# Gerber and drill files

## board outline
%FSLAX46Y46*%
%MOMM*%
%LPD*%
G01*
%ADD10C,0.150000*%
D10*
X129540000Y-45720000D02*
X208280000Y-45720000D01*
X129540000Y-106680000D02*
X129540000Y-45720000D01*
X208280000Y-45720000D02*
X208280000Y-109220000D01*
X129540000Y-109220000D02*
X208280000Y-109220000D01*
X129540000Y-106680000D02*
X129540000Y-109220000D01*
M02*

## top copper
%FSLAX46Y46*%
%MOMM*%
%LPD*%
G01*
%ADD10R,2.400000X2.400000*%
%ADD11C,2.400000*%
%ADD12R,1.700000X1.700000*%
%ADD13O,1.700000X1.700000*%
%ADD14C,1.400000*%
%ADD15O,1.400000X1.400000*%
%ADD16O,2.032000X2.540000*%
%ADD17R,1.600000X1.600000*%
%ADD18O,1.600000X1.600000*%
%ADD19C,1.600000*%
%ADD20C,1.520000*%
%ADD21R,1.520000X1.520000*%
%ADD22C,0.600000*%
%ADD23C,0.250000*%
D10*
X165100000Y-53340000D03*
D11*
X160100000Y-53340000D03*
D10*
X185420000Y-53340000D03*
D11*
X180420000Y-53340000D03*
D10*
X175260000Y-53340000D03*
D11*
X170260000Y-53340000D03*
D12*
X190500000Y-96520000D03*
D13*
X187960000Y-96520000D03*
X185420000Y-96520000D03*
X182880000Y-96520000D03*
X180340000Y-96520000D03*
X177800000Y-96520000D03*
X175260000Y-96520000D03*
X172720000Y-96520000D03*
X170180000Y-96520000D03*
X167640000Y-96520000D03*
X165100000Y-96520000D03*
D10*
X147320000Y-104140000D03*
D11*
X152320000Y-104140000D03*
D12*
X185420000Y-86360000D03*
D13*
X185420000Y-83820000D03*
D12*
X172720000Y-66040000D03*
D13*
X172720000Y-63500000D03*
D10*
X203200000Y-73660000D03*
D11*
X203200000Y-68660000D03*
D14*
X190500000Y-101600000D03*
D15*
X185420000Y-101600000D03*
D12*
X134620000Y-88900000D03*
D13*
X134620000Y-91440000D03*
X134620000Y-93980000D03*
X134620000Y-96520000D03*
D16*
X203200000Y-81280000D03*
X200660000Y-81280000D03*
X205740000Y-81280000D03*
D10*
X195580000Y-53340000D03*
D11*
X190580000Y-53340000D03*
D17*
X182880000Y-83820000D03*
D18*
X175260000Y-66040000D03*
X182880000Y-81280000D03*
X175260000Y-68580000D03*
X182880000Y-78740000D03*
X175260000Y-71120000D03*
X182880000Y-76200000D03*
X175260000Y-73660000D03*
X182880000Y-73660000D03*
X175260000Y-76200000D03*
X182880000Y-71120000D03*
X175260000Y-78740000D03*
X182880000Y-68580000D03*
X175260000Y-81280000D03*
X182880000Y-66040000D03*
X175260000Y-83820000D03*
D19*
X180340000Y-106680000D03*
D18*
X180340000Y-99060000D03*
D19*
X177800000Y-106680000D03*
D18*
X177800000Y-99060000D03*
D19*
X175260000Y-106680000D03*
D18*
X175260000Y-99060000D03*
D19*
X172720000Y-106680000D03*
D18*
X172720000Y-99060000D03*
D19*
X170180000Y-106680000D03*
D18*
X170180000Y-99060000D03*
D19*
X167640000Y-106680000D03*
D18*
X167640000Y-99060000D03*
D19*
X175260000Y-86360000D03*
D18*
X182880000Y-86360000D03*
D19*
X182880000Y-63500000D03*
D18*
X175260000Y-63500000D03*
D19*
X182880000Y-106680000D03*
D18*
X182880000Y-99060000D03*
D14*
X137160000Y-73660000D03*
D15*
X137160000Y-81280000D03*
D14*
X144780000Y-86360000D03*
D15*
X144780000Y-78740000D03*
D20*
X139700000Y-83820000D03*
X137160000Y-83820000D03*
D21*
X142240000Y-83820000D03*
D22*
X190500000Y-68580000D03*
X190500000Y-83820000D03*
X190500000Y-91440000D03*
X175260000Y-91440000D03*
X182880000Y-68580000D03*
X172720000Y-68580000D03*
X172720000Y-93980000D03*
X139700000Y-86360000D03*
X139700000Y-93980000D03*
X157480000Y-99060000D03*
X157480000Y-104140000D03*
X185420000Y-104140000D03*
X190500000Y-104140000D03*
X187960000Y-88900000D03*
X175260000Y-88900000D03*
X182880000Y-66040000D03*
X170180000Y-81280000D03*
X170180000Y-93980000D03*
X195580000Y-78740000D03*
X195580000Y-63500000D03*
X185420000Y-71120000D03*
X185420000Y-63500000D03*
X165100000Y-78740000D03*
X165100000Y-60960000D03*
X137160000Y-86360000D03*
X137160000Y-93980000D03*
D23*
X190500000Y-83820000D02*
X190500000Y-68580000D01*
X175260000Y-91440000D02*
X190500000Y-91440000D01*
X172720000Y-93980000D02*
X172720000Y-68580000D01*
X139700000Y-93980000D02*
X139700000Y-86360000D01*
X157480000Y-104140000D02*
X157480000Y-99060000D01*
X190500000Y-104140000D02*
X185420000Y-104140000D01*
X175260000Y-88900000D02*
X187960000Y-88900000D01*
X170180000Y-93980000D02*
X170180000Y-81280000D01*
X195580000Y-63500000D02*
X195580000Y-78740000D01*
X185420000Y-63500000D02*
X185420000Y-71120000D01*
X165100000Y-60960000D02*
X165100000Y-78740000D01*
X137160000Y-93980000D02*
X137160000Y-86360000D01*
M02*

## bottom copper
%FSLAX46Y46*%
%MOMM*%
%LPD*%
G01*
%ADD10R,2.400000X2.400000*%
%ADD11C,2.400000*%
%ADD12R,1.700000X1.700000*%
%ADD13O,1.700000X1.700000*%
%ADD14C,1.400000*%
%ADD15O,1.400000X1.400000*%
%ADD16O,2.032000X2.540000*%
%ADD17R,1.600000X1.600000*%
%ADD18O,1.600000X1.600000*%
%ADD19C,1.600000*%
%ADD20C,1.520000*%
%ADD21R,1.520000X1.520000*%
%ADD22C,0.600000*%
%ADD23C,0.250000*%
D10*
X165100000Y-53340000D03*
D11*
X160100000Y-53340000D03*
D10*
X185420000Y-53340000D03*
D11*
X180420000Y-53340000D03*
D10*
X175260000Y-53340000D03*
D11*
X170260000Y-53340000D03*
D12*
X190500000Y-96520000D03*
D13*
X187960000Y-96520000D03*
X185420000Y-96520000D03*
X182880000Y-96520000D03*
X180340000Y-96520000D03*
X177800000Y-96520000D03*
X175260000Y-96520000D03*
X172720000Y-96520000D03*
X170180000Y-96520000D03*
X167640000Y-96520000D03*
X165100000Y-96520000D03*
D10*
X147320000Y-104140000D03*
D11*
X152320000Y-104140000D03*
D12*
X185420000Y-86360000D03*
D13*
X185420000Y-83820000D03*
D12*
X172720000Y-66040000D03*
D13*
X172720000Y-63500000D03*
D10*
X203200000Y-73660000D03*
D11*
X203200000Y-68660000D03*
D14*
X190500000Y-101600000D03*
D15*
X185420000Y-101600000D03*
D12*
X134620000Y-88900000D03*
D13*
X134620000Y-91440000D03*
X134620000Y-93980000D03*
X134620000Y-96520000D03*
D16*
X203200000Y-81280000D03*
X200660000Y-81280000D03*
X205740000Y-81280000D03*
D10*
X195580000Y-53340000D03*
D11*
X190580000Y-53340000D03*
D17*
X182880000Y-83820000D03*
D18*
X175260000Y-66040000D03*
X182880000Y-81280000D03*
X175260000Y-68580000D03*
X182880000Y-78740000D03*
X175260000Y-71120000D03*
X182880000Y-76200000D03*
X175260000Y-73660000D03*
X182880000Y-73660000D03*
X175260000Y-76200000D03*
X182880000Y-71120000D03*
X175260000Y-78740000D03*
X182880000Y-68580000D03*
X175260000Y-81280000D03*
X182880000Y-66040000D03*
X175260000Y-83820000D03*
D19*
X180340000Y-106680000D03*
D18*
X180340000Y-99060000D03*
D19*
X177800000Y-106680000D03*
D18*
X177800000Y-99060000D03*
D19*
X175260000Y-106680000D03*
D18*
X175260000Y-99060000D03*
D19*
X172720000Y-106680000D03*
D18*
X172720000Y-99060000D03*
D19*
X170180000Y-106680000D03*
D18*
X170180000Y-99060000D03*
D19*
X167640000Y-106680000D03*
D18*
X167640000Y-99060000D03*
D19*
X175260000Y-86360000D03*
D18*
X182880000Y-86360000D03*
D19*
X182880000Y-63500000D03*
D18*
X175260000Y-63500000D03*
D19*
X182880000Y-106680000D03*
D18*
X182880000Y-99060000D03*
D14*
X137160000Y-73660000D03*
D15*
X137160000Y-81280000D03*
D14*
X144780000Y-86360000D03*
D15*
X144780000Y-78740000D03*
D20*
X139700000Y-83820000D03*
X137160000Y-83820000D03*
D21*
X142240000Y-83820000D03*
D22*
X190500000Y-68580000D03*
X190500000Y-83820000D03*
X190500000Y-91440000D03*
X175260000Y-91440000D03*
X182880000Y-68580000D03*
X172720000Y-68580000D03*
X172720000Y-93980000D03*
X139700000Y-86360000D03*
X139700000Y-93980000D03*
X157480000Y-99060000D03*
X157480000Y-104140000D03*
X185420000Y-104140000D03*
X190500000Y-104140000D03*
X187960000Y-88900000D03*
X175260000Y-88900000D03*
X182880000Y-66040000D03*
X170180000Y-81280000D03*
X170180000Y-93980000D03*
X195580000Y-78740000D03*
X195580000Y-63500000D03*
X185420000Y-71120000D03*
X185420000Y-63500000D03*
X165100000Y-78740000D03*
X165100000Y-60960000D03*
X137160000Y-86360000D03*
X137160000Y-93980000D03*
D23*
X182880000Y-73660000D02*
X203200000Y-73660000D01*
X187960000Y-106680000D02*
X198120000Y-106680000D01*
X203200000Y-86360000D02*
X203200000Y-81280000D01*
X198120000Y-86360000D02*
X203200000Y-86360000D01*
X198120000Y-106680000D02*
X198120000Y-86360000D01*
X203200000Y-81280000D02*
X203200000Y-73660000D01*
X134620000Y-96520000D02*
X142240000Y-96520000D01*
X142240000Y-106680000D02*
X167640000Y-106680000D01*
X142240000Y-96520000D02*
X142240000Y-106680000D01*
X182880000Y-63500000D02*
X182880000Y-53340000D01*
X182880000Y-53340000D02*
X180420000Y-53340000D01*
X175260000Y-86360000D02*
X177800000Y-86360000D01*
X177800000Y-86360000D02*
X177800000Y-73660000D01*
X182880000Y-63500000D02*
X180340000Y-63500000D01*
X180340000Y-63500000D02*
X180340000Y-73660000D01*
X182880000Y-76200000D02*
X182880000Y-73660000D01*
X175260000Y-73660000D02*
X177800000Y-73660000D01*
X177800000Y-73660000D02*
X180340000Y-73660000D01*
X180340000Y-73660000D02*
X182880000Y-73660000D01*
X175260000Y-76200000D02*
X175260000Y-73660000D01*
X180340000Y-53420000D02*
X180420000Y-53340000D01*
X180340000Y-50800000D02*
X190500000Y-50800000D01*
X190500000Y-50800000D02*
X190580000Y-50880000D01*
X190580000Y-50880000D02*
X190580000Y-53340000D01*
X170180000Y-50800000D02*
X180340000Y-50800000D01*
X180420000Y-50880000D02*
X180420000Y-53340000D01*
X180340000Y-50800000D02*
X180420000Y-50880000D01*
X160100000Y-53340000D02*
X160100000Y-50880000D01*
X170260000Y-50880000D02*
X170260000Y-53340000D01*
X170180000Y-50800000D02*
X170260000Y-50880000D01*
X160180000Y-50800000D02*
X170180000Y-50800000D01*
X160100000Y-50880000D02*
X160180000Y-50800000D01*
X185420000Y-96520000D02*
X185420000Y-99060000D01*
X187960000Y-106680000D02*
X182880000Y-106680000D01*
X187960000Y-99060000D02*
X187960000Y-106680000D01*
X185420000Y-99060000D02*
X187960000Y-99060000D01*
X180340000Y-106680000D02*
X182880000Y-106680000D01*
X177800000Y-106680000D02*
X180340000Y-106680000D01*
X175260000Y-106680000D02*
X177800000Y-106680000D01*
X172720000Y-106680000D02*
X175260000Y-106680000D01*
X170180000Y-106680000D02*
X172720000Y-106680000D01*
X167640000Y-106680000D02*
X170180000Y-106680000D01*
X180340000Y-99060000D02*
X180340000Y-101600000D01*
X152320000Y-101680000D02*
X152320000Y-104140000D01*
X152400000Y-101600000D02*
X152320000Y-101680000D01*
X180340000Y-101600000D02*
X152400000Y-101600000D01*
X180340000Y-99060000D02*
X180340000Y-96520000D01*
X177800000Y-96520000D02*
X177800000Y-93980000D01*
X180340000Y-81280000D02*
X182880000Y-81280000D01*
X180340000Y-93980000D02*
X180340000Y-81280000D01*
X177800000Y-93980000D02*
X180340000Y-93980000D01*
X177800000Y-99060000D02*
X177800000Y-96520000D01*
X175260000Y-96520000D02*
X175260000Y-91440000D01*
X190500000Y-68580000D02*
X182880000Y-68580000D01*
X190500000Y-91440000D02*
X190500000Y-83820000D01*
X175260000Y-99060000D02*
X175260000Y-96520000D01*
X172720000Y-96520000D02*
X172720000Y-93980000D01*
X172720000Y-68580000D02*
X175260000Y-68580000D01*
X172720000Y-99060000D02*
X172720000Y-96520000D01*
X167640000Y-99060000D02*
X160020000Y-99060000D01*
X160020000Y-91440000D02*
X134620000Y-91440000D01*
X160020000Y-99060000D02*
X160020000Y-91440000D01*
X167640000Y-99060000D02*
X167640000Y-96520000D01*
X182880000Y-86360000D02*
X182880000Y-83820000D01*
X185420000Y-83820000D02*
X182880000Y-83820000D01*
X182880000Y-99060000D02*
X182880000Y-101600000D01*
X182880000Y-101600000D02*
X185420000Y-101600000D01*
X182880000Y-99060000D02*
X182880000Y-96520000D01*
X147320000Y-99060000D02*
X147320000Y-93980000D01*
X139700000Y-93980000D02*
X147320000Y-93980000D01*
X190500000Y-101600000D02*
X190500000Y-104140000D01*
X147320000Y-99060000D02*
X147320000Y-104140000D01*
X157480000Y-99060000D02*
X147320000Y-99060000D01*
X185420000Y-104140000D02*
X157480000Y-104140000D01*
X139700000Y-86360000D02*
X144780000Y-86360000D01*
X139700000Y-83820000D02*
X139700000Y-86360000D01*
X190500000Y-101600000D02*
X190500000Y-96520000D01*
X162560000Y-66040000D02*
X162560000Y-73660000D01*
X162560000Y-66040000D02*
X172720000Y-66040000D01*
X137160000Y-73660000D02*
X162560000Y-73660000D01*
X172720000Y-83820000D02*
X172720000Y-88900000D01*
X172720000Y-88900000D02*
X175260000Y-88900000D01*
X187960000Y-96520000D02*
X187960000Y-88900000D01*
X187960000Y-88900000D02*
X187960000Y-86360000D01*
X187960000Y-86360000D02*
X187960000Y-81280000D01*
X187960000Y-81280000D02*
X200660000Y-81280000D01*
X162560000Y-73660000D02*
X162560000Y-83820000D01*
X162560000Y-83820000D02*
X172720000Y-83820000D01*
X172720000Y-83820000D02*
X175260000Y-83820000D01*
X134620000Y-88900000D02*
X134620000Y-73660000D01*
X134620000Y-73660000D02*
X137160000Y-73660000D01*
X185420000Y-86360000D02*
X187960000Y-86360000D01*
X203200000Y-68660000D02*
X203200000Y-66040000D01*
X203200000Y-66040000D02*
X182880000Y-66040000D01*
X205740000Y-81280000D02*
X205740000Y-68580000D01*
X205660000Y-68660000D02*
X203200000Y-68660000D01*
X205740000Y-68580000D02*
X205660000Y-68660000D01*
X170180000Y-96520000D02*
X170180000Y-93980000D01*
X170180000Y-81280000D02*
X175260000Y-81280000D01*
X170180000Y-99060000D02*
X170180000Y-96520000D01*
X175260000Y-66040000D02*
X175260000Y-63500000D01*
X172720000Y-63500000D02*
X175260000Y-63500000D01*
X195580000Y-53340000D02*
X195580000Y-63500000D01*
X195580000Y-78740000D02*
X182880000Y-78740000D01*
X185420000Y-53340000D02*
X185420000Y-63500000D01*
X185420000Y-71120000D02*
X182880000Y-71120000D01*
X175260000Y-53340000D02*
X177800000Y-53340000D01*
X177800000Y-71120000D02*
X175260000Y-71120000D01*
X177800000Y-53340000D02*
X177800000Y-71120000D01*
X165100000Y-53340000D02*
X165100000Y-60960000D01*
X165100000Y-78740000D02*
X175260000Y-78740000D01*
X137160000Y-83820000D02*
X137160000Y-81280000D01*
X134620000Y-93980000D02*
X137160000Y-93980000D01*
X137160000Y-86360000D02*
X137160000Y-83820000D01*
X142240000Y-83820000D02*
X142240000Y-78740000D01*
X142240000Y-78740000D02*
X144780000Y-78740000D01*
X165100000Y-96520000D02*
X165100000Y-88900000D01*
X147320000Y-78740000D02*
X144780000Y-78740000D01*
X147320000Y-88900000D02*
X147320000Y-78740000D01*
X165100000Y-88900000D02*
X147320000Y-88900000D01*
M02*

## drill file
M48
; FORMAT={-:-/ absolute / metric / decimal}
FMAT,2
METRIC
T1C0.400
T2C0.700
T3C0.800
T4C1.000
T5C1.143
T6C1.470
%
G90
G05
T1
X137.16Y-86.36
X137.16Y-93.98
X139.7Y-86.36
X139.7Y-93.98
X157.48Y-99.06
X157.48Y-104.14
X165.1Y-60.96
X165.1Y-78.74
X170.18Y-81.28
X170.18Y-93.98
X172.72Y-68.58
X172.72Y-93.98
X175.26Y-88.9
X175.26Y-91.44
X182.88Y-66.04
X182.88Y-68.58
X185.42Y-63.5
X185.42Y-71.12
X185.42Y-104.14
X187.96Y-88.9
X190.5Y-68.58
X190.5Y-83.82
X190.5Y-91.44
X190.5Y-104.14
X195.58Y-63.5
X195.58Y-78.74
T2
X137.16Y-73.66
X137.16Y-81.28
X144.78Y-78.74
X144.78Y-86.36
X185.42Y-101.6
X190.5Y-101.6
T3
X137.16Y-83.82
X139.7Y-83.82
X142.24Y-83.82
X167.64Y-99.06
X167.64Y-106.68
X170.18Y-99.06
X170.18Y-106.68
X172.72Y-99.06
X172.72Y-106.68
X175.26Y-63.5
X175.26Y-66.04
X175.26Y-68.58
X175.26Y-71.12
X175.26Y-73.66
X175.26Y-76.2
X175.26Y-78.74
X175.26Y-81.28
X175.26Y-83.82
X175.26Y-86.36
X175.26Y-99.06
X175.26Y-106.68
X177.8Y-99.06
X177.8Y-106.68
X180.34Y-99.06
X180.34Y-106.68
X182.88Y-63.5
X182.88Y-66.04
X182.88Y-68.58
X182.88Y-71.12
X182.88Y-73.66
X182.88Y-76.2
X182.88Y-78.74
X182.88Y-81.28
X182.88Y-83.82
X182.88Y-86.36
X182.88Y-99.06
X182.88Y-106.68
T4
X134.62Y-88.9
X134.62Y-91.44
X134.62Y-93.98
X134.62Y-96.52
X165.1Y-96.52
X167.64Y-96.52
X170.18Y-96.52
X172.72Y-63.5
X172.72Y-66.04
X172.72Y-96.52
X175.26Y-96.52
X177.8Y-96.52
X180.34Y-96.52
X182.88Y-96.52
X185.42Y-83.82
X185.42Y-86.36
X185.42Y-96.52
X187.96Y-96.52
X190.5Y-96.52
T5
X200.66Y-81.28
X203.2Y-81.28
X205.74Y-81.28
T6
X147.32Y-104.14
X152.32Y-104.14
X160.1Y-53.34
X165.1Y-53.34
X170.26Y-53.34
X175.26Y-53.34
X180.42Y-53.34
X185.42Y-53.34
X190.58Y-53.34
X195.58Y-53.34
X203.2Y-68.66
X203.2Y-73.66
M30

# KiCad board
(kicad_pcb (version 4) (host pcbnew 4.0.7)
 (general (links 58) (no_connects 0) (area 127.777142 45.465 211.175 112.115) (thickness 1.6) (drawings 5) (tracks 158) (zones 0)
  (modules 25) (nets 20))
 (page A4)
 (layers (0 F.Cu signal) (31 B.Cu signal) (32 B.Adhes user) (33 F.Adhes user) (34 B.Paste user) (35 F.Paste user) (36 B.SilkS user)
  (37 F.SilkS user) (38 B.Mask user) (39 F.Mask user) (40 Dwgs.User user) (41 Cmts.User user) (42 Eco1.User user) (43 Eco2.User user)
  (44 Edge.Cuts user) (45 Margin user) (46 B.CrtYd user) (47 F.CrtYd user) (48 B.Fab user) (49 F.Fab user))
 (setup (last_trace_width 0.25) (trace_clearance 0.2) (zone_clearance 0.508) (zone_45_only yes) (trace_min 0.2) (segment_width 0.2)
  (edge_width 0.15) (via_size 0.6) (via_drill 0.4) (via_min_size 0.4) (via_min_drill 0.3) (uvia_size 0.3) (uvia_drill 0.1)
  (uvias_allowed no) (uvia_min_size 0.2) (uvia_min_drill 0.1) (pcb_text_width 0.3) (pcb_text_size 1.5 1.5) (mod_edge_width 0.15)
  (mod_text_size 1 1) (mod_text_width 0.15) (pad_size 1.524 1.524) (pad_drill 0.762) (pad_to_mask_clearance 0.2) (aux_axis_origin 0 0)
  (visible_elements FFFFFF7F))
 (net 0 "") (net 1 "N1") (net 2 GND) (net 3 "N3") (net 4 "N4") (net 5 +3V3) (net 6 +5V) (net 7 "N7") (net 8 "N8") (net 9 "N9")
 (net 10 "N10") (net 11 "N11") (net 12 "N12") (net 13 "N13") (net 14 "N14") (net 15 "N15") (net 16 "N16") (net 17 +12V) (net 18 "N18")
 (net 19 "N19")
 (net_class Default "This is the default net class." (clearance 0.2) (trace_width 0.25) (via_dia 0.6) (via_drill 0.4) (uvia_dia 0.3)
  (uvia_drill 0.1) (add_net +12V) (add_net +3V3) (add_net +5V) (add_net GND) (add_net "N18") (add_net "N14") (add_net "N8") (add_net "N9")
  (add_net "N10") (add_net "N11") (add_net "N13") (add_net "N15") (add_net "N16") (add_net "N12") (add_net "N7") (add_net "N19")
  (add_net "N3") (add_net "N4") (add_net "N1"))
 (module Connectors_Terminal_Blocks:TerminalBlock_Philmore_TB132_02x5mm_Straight (layer F.Cu) (at 165.1 53.34 180)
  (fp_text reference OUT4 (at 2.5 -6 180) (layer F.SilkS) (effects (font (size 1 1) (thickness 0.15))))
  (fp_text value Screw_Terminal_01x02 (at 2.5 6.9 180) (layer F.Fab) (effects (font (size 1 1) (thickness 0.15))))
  (pad 1 thru_hole rect (at 0 0 180) (size 2.4 2.4) (drill 1.47) (layers *.Cu *.Mask) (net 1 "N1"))
  (pad 2 thru_hole circle (at 5 0 180) (size 2.4 2.4) (drill 1.47) (layers *.Cu *.Mask) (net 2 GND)))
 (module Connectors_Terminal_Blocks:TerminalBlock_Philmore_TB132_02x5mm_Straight (layer F.Cu) (at 185.42 53.34 180)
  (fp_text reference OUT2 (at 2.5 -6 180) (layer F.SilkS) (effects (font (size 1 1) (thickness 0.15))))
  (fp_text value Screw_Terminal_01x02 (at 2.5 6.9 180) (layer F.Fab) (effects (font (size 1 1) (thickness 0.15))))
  (pad 1 thru_hole rect (at 0 0 180) (size 2.4 2.4) (drill 1.47) (layers *.Cu *.Mask) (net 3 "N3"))
  (pad 2 thru_hole circle (at 5 0 180) (size 2.4 2.4) (drill 1.47) (layers *.Cu *.Mask) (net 2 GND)))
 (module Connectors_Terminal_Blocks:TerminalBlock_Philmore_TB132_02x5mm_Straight (layer F.Cu) (at 175.26 53.34 180)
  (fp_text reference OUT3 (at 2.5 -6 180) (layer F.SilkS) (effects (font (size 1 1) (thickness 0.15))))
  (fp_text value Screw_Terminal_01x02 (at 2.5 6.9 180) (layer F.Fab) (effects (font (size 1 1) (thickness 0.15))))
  (pad 1 thru_hole rect (at 0 0 180) (size 2.4 2.4) (drill 1.47) (layers *.Cu *.Mask) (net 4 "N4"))
  (pad 2 thru_hole circle (at 5 0 180) (size 2.4 2.4) (drill 1.47) (layers *.Cu *.Mask) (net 2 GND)))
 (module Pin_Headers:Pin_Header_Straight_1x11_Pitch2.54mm (layer F.Cu) (at 190.5 96.52 270)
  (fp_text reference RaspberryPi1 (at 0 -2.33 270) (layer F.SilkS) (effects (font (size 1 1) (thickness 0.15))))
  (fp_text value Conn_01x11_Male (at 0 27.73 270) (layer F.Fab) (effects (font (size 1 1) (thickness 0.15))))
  (pad 1 thru_hole rect (at 0 0 270) (size 1.7 1.7) (drill 1) (layers *.Cu *.Mask) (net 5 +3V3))
  (pad 2 thru_hole oval (at 0 2.54 270) (size 1.7 1.7) (drill 1) (layers *.Cu *.Mask) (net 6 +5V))
  (pad 3 thru_hole oval (at 0 5.08 270) (size 1.7 1.7) (drill 1) (layers *.Cu *.Mask) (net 2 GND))
  (pad 4 thru_hole oval (at 0 7.62 270) (size 1.7 1.7) (drill 1) (layers *.Cu *.Mask) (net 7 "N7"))
  (pad 5 thru_hole oval (at 0 10.16 270) (size 1.7 1.7) (drill 1) (layers *.Cu *.Mask) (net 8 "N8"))
  (pad 6 thru_hole oval (at 0 12.7 270) (size 1.7 1.7) (drill 1) (layers *.Cu *.Mask) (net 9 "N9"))
  (pad 7 thru_hole oval (at 0 15.24 270) (size 1.7 1.7) (drill 1) (layers *.Cu *.Mask) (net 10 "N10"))
  (pad 8 thru_hole oval (at 0 17.78 270) (size 1.7 1.7) (drill 1) (layers *.Cu *.Mask) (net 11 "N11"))
  (pad 9 thru_hole oval (at 0 20.32 270) (size 1.7 1.7) (drill 1) (layers *.Cu *.Mask) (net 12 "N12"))
  (pad 10 thru_hole oval (at 0 22.86 270) (size 1.7 1.7) (drill 1) (layers *.Cu *.Mask) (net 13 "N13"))
  (pad 11 thru_hole oval (at 0 25.4 270) (size 1.7 1.7) (drill 1) (layers *.Cu *.Mask) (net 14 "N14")))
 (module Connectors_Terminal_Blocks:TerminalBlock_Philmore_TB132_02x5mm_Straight (layer F.Cu) (at 147.32 104.14)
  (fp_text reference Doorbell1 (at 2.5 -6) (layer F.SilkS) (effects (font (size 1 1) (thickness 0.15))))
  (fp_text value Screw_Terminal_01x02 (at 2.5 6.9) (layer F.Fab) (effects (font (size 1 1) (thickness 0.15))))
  (pad 1 thru_hole rect (at 0 0) (size 2.4 2.4) (drill 1.47) (layers *.Cu *.Mask) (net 5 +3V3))
  (pad 2 thru_hole circle (at 5 0) (size 2.4 2.4) (drill 1.47) (layers *.Cu *.Mask) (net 8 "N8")))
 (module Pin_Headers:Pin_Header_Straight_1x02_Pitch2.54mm (layer F.Cu) (at 185.42 86.36 180)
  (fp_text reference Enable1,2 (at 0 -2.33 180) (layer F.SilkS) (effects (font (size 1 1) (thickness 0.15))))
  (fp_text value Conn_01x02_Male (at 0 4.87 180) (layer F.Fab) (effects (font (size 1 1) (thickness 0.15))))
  (pad 1 thru_hole rect (at 0 0 180) (size 1.7 1.7) (drill 1) (layers *.Cu *.Mask) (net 6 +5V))
  (pad 2 thru_hole oval (at 0 2.54 180) (size 1.7 1.7) (drill 1) (layers *.Cu *.Mask) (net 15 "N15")))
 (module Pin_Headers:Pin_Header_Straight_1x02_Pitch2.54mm (layer F.Cu) (at 172.72 66.04 180)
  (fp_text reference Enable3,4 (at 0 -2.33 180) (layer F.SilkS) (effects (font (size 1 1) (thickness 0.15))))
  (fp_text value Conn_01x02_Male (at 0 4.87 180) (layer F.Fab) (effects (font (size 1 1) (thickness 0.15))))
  (pad 1 thru_hole rect (at 0 0 180) (size 1.7 1.7) (drill 1) (layers *.Cu *.Mask) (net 6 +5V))
  (pad 2 thru_hole oval (at 0 2.54 180) (size 1.7 1.7) (drill 1) (layers *.Cu *.Mask) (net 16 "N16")))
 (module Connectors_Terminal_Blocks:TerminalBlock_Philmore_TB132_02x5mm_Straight (layer F.Cu) (at 203.2 73.66 90)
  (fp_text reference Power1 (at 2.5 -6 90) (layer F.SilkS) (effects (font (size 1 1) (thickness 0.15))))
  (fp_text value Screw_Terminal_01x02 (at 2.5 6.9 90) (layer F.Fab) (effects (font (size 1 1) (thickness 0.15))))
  (pad 1 thru_hole rect (at 0 0 90) (size 2.4 2.4) (drill 1.47) (layers *.Cu *.Mask) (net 2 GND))
  (pad 2 thru_hole circle (at 5 0 90) (size 2.4 2.4) (drill 1.47) (layers *.Cu *.Mask) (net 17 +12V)))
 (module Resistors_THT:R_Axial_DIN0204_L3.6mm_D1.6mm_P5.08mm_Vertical (layer F.Cu) (at 190.5 101.6 180)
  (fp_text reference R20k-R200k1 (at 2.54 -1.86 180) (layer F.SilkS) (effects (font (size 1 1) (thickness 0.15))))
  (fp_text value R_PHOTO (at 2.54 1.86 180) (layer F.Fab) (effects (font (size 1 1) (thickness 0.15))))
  (pad 1 thru_hole circle (at 0 0 180) (size 1.4 1.4) (drill 0.7) (layers *.Cu *.Mask) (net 5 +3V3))
  (pad 2 thru_hole oval (at 5.08 0 180) (size 1.4 1.4) (drill 0.7) (layers *.Cu *.Mask) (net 7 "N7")))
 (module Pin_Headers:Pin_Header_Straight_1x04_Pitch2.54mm (layer F.Cu) (at 134.62 88.9)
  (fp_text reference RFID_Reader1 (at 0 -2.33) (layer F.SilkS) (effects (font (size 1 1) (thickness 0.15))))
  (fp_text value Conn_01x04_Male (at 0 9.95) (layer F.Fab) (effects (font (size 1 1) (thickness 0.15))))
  (pad 1 thru_hole rect (at 0 0) (size 1.7 1.7) (drill 1) (layers *.Cu *.Mask) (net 6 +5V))
  (pad 2 thru_hole oval (at 0 2.54) (size 1.7 1.7) (drill 1) (layers *.Cu *.Mask) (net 13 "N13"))
  (pad 3 thru_hole oval (at 0 5.08) (size 1.7 1.7) (drill 1) (layers *.Cu *.Mask) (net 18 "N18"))
  (pad 4 thru_hole oval (at 0 7.62) (size 1.7 1.7) (drill 1) (layers *.Cu *.Mask) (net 2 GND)))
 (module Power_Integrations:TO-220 (layer F.Cu) (at 203.2 81.28 180)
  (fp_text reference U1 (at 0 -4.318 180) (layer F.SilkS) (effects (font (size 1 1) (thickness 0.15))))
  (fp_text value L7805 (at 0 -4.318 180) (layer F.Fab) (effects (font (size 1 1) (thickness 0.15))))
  (pad 2 thru_hole oval (at 0 0 180) (size 2.032 2.54) (drill 1.143) (layers *.Cu *.Mask) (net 2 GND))
  (pad 3 thru_hole oval (at 2.54 0 180) (size 2.032 2.54) (drill 1.143) (layers *.Cu *.Mask) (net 6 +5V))
  (pad 1 thru_hole oval (at -2.54 0 180) (size 2.032 2.54) (drill 1.143) (layers *.Cu *.Mask) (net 17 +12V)))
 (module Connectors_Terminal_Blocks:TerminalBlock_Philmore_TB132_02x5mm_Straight (layer F.Cu) (at 195.58 53.34 180)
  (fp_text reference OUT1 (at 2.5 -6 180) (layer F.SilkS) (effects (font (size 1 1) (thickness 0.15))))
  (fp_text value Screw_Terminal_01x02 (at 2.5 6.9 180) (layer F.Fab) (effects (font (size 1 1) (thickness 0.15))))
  (pad 1 thru_hole rect (at 0 0 180) (size 2.4 2.4) (drill 1.47) (layers *.Cu *.Mask) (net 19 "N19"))
  (pad 2 thru_hole circle (at 5 0 180) (size 2.4 2.4) (drill 1.47) (layers *.Cu *.Mask) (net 2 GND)))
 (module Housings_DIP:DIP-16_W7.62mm (layer F.Cu) (at 182.88 83.82 180)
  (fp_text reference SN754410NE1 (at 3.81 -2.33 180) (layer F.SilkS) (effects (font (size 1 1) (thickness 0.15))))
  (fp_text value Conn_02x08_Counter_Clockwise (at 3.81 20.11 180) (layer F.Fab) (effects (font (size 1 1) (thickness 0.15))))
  (pad 1 thru_hole rect (at 0 0 180) (size 1.6 1.6) (drill 0.8) (layers *.Cu *.Mask) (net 15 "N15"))
  (pad 9 thru_hole oval (at 7.62 17.78 180) (size 1.6 1.6) (drill 0.8) (layers *.Cu *.Mask) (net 16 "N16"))
  (pad 2 thru_hole oval (at 0 2.54 180) (size 1.6 1.6) (drill 0.8) (layers *.Cu *.Mask) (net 9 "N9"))
  (pad 10 thru_hole oval (at 7.62 15.24 180) (size 1.6 1.6) (drill 0.8) (layers *.Cu *.Mask) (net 11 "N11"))
  (pad 3 thru_hole oval (at 0 5.08 180) (size 1.6 1.6) (drill 0.8) (layers *.Cu *.Mask) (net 19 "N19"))
  (pad 11 thru_hole oval (at 7.62 12.7 180) (size 1.6 1.6) (drill 0.8) (layers *.Cu *.Mask) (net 4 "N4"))
  (pad 4 thru_hole oval (at 0 7.62 180) (size 1.6 1.6) (drill 0.8) (layers *.Cu *.Mask) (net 2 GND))
  (pad 12 thru_hole oval (at 7.62 10.16 180) (size 1.6 1.6) (drill 0.8) (layers *.Cu *.Mask) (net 2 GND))
  (pad 5 thru_hole oval (at 0 10.16 180) (size 1.6 1.6) (drill 0.8) (layers *.Cu *.Mask) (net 2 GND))
  (pad 13 thru_hole oval (at 7.62 7.62 180) (size 1.6 1.6) (drill 0.8) (layers *.Cu *.Mask) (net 2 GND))
  (pad 6 thru_hole oval (at 0 12.7 180) (size 1.6 1.6) (drill 0.8) (layers *.Cu *.Mask) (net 3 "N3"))
  (pad 14 thru_hole oval (at 7.62 5.08 180) (size 1.6 1.6) (drill 0.8) (layers *.Cu *.Mask) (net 1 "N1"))
  (pad 7 thru_hole oval (at 0 15.24 180) (size 1.6 1.6) (drill 0.8) (layers *.Cu *.Mask) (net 10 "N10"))
  (pad 15 thru_hole oval (at 7.62 2.54 180) (size 1.6 1.6) (drill 0.8) (layers *.Cu *.Mask) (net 12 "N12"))
  (pad 8 thru_hole oval (at 0 17.78 180) (size 1.6 1.6) (drill 0.8) (layers *.Cu *.Mask) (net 17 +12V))
  (pad 16 thru_hole oval (at 7.62 0 180) (size 1.6 1.6) (drill 0.8) (layers *.Cu *.Mask) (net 6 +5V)))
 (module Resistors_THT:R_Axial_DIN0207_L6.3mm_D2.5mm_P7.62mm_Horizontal (layer F.Cu) (at 180.34 106.68 90)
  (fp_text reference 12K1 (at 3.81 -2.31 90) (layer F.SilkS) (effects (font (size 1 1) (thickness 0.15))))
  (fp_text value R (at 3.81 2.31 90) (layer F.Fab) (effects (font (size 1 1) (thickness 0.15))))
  (pad 1 thru_hole circle (at 0 0 90) (size 1.6 1.6) (drill 0.8) (layers *.Cu *.Mask) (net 2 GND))
  (pad 2 thru_hole oval (at 7.62 0 90) (size 1.6 1.6) (drill 0.8) (layers *.Cu *.Mask) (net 8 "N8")))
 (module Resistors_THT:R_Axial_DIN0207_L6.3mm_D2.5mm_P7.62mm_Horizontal (layer F.Cu) (at 177.8 106.68 90)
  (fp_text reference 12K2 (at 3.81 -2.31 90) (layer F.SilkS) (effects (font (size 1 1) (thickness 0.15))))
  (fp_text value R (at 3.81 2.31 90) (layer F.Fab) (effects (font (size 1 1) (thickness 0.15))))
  (pad 1 thru_hole circle (at 0 0 90) (size 1.6 1.6) (drill 0.8) (layers *.Cu *.Mask) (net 2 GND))
  (pad 2 thru_hole oval (at 7.62 0 90) (size 1.6 1.6) (drill 0.8) (layers *.Cu *.Mask) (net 9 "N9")))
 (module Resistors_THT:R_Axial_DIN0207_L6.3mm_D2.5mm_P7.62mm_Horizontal (layer F.Cu) (at 175.26 106.68 90)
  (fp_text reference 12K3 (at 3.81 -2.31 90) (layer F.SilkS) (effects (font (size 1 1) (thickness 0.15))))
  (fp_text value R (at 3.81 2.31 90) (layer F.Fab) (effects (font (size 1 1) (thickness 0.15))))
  (pad 1 thru_hole circle (at 0 0 90) (size 1.6 1.6) (drill 0.8) (layers *.Cu *.Mask) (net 2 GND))
  (pad 2 thru_hole oval (at 7.62 0 90) (size 1.6 1.6) (drill 0.8) (layers *.Cu *.Mask) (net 10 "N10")))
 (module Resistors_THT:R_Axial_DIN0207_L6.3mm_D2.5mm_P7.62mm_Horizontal (layer F.Cu) (at 172.72 106.68 90)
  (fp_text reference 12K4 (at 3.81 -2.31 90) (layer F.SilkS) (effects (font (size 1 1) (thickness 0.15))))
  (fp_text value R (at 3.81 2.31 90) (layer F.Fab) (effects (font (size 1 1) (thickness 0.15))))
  (pad 1 thru_hole circle (at 0 0 90) (size 1.6 1.6) (drill 0.8) (layers *.Cu *.Mask) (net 2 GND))
  (pad 2 thru_hole oval (at 7.62 0 90) (size 1.6 1.6) (drill 0.8) (layers *.Cu *.Mask) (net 11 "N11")))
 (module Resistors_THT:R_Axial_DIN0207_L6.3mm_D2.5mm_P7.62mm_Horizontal (layer F.Cu) (at 170.18 106.68 90)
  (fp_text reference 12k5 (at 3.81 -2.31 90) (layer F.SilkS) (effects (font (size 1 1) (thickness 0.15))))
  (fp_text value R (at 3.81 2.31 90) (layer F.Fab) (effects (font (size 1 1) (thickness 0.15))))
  (pad 1 thru_hole circle (at 0 0 90) (size 1.6 1.6) (drill 0.8) (layers *.Cu *.Mask) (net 2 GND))
  (pad 2 thru_hole oval (at 7.62 0 90) (size 1.6 1.6) (drill 0.8) (layers *.Cu *.Mask) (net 12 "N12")))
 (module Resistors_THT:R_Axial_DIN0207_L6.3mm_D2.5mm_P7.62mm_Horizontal (layer F.Cu) (at 167.64 106.68 90)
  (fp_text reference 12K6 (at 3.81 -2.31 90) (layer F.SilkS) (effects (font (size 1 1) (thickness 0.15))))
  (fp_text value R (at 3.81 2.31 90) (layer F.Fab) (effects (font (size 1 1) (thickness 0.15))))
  (pad 1 thru_hole circle (at 0 0 90) (size 1.6 1.6) (drill 0.8) (layers *.Cu *.Mask) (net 2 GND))
  (pad 2 thru_hole oval (at 7.62 0 90) (size 1.6 1.6) (drill 0.8) (layers *.Cu *.Mask) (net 13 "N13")))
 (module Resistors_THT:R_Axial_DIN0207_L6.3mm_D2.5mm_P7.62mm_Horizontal (layer F.Cu) (at 175.26 86.36)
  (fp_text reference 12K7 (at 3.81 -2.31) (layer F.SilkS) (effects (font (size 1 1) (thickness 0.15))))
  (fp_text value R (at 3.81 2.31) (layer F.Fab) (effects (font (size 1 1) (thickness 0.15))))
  (pad 1 thru_hole circle (at 0 0) (size 1.6 1.6) (drill 0.8) (layers *.Cu *.Mask) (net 2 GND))
  (pad 2 thru_hole oval (at 7.62 0) (size 1.6 1.6) (drill 0.8) (layers *.Cu *.Mask) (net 15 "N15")))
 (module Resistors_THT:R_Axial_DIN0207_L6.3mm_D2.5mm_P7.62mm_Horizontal (layer F.Cu) (at 182.88 63.5 180)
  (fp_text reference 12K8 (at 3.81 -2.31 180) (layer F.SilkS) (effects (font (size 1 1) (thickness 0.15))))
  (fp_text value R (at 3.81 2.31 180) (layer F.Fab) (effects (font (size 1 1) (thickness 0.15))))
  (pad 1 thru_hole circle (at 0 0 180) (size 1.6 1.6) (drill 0.8) (layers *.Cu *.Mask) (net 2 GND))
  (pad 2 thru_hole oval (at 7.62 0 180) (size 1.6 1.6) (drill 0.8) (layers *.Cu *.Mask) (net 16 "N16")))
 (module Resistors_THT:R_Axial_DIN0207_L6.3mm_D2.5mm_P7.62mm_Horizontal (layer F.Cu) (at 182.88 106.68 90)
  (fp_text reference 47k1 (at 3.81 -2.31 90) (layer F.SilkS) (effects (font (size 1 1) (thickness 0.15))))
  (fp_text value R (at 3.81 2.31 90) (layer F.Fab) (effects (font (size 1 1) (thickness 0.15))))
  (pad 1 thru_hole circle (at 0 0 90) (size 1.6 1.6) (drill 0.8) (layers *.Cu *.Mask) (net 2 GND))
  (pad 2 thru_hole oval (at 7.62 0 90) (size 1.6 1.6) (drill 0.8) (layers *.Cu *.Mask) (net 7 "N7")))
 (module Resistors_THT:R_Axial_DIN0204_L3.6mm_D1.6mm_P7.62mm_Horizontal (layer F.Cu) (at 137.16 73.66 270)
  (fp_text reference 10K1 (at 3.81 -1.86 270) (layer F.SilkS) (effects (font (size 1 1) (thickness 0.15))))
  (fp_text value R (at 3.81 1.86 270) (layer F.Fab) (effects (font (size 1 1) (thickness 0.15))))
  (pad 1 thru_hole circle (at 0 0 270) (size 1.4 1.4) (drill 0.7) (layers *.Cu *.Mask) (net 6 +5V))
  (pad 2 thru_hole oval (at 7.62 0 270) (size 1.4 1.4) (drill 0.7) (layers *.Cu *.Mask) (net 18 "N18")))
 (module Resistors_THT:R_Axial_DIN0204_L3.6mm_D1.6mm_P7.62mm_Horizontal (layer F.Cu) (at 144.78 86.36 90)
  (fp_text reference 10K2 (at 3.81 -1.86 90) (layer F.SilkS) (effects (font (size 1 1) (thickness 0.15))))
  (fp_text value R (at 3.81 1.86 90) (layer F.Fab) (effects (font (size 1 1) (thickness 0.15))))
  (pad 1 thru_hole circle (at 0 0 90) (size 1.4 1.4) (drill 0.7) (layers *.Cu *.Mask) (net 5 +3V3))
  (pad 2 thru_hole oval (at 7.62 0 90) (size 1.4 1.4) (drill 0.7) (layers *.Cu *.Mask) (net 14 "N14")))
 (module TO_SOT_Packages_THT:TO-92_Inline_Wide (layer F.Cu) (at 142.24 83.82 180)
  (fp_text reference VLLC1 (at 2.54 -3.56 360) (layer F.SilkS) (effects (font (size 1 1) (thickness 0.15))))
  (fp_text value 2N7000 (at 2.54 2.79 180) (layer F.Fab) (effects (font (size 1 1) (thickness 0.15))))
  (pad 2 thru_hole circle (at 2.54 0 270) (size 1.52 1.52) (drill 0.8) (layers *.Cu *.Mask) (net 5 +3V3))
  (pad 3 thru_hole circle (at 5.08 0 270) (size 1.52 1.52) (drill 0.8) (layers *.Cu *.Mask) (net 18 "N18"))
  (pad 1 thru_hole rect (at 0 0 270) (size 1.52 1.52) (drill 0.8) (layers *.Cu *.Mask) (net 14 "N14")))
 (gr_line (start 129.54 45.72) (end 208.28 45.72) (angle 90) (layer Edge.Cuts) (width 0.15))
 (gr_line (start 129.54 106.68) (end 129.54 45.72) (angle 90) (layer Edge.Cuts) (width 0.15))
 (gr_line (start 208.28 45.72) (end 208.28 109.22) (angle 90) (layer Edge.Cuts) (width 0.15))
 (gr_line (start 129.54 109.22) (end 208.28 109.22) (angle 90) (layer Edge.Cuts) (width 0.15))
 (gr_line (start 129.54 106.68) (end 129.54 109.22) (angle 90) (layer Edge.Cuts) (width 0.15))
 (segment (start 182.88 73.66) (end 203.2 73.66) (width 0.25) (layer B.Cu) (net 2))
 (segment (start 187.96 106.68) (end 198.12 106.68) (width 0.25) (layer B.Cu) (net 2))
 (segment (start 203.2 86.36) (end 203.2 81.28) (width 0.25) (layer B.Cu) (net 2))
 (segment (start 198.12 86.36) (end 203.2 86.36) (width 0.25) (layer B.Cu) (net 2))
 (segment (start 198.12 106.68) (end 198.12 86.36) (width 0.25) (layer B.Cu) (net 2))
 (segment (start 203.2 81.28) (end 203.2 73.66) (width 0.25) (layer B.Cu) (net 2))
 (segment (start 134.62 96.52) (end 142.24 96.52) (width 0.25) (layer B.Cu) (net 2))
 (segment (start 142.24 106.68) (end 167.64 106.68) (width 0.25) (layer B.Cu) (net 2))
 (segment (start 142.24 96.52) (end 142.24 106.68) (width 0.25) (layer B.Cu) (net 2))
 (segment (start 182.88 63.5) (end 182.88 53.34) (width 0.25) (layer B.Cu) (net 2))
 (segment (start 182.88 53.34) (end 180.42 53.34) (width 0.25) (layer B.Cu) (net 2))
 (segment (start 175.26 86.36) (end 177.8 86.36) (width 0.25) (layer B.Cu) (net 2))
 (segment (start 177.8 86.36) (end 177.8 73.66) (width 0.25) (layer B.Cu) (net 2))
 (segment (start 182.88 63.5) (end 180.34 63.5) (width 0.25) (layer B.Cu) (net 2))
 (segment (start 180.34 63.5) (end 180.34 73.66) (width 0.25) (layer B.Cu) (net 2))
 (segment (start 182.88 76.2) (end 182.88 73.66) (width 0.25) (layer B.Cu) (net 2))
 (segment (start 175.26 73.66) (end 177.8 73.66) (width 0.25) (layer B.Cu) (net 2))
 (segment (start 177.8 73.66) (end 180.34 73.66) (width 0.25) (layer B.Cu) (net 2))
 (segment (start 180.34 73.66) (end 182.88 73.66) (width 0.25) (layer B.Cu) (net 2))
 (segment (start 175.26 76.2) (end 175.26 73.66) (width 0.25) (layer B.Cu) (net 2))
 (segment (start 180.34 53.42) (end 180.42 53.34) (width 0.25) (layer B.Cu) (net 2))
 (segment (start 180.34 50.8) (end 190.5 50.8) (width 0.25) (layer B.Cu) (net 2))
 (segment (start 190.5 50.8) (end 190.58 50.88) (width 0.25) (layer B.Cu) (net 2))
 (segment (start 190.58 50.88) (end 190.58 53.34) (width 0.25) (layer B.Cu) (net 2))
 (segment (start 170.18 50.8) (end 180.34 50.8) (width 0.25) (layer B.Cu) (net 2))
 (segment (start 180.42 50.88) (end 180.42 53.34) (width 0.25) (layer B.Cu) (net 2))
 (segment (start 180.34 50.8) (end 180.42 50.88) (width 0.25) (layer B.Cu) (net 2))
 (segment (start 160.1 53.34) (end 160.1 50.88) (width 0.25) (layer B.Cu) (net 2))
 (segment (start 170.26 50.88) (end 170.26 53.34) (width 0.25) (layer B.Cu) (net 2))
 (segment (start 170.18 50.8) (end 170.26 50.88) (width 0.25) (layer B.Cu) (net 2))
 (segment (start 160.18 50.8) (end 170.18 50.8) (width 0.25) (layer B.Cu) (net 2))
 (segment (start 160.1 50.88) (end 160.18 50.8) (width 0.25) (layer B.Cu) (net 2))
 (segment (start 185.42 96.52) (end 185.42 99.06) (width 0.25) (layer B.Cu) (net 2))
 (segment (start 187.96 106.68) (end 182.88 106.68) (width 0.25) (layer B.Cu) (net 2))
 (segment (start 187.96 99.06) (end 187.96 106.68) (width 0.25) (layer B.Cu) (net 2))
 (segment (start 185.42 99.06) (end 187.96 99.06) (width 0.25) (layer B.Cu) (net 2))
 (segment (start 180.34 106.68) (end 182.88 106.68) (width 0.25) (layer B.Cu) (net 2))
 (segment (start 177.8 106.68) (end 180.34 106.68) (width 0.25) (layer B.Cu) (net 2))
 (segment (start 175.26 106.68) (end 177.8 106.68) (width 0.25) (layer B.Cu) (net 2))
 (segment (start 172.72 106.68) (end 175.26 106.68) (width 0.25) (layer B.Cu) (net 2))
 (segment (start 170.18 106.68) (end 172.72 106.68) (width 0.25) (layer B.Cu) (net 2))
 (segment (start 167.64 106.68) (end 170.18 106.68) (width 0.25) (layer B.Cu) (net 2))
 (segment (start 180.34 99.06) (end 180.34 101.6) (width 0.25) (layer B.Cu) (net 8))
 (segment (start 152.32 101.68) (end 152.32 104.14) (width 0.25) (layer B.Cu) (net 8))
 (segment (start 152.4 101.6) (end 152.32 101.68) (width 0.25) (layer B.Cu) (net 8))
 (segment (start 180.34 101.6) (end 152.4 101.6) (width 0.25) (layer B.Cu) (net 8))
 (segment (start 180.34 99.06) (end 180.34 96.52) (width 0.25) (layer B.Cu) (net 8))
 (segment (start 177.8 96.52) (end 177.8 93.98) (width 0.25) (layer B.Cu) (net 9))
 (segment (start 180.34 81.28) (end 182.88 81.28) (width 0.25) (layer B.Cu) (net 9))
 (segment (start 180.34 93.98) (end 180.34 81.28) (width 0.25) (layer B.Cu) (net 9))
 (segment (start 177.8 93.98) (end 180.34 93.98) (width 0.25) (layer B.Cu) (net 9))
 (segment (start 177.8 99.06) (end 177.8 96.52) (width 0.25) (layer B.Cu) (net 9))
 (segment (start 175.26 96.52) (end 175.26 91.44) (width 0.25) (layer B.Cu) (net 10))
 (segment (start 190.5 68.58) (end 182.88 68.58) (width 0.25) (layer B.Cu) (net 10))
 (via (at 190.5 68.58) (size 0.6) (drill 0.4) (layers F.Cu B.Cu) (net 10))
 (segment (start 190.5 83.82) (end 190.5 68.58) (width 0.25) (layer F.Cu) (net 10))
 (via (at 190.5 83.82) (size 0.6) (drill 0.4) (layers F.Cu B.Cu) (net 10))
 (segment (start 190.5 91.44) (end 190.5 83.82) (width 0.25) (layer B.Cu) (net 10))
 (via (at 190.5 91.44) (size 0.6) (drill 0.4) (layers F.Cu B.Cu) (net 10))
 (segment (start 175.26 91.44) (end 190.5 91.44) (width 0.25) (layer F.Cu) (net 10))
 (via (at 175.26 91.44) (size 0.6) (drill 0.4) (layers F.Cu B.Cu) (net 10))
 (via (at 182.88 68.58) (size 0.6) (drill 0.4) (layers F.Cu B.Cu) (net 10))
 (segment (start 175.26 99.06) (end 175.26 96.52) (width 0.25) (layer B.Cu) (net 10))
 (segment (start 172.72 96.52) (end 172.72 93.98) (width 0.25) (layer B.Cu) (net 11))
 (segment (start 172.72 68.58) (end 175.26 68.58) (width 0.25) (layer B.Cu) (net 11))
 (via (at 172.72 68.58) (size 0.6) (drill 0.4) (layers F.Cu B.Cu) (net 11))
 (segment (start 172.72 93.98) (end 172.72 68.58) (width 0.25) (layer F.Cu) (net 11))
 (via (at 172.72 93.98) (size 0.6) (drill 0.4) (layers F.Cu B.Cu) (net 11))
 (segment (start 172.72 99.06) (end 172.72 96.52) (width 0.25) (layer B.Cu) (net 11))
 (segment (start 167.64 99.06) (end 160.02 99.06) (width 0.25) (layer B.Cu) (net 13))
 (segment (start 160.02 91.44) (end 134.62 91.44) (width 0.25) (layer B.Cu) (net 13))
 (segment (start 160.02 99.06) (end 160.02 91.44) (width 0.25) (layer B.Cu) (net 13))
 (segment (start 167.64 99.06) (end 167.64 96.52) (width 0.25) (layer B.Cu) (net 13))
 (segment (start 182.88 86.36) (end 182.88 83.82) (width 0.25) (layer B.Cu) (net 15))
 (segment (start 185.42 83.82) (end 182.88 83.82) (width 0.25) (layer B.Cu) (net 15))
 (segment (start 182.88 99.06) (end 182.88 101.6) (width 0.25) (layer B.Cu) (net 7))
 (segment (start 182.88 101.6) (end 185.42 101.6) (width 0.25) (layer B.Cu) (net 7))
 (segment (start 182.88 99.06) (end 182.88 96.52) (width 0.25) (layer B.Cu) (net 7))
 (via (at 139.7 86.36) (size 0.6) (drill 0.4) (layers F.Cu B.Cu) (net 5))
 (segment (start 147.32 99.06) (end 147.32 93.98) (width 0.25) (layer B.Cu) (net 5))
 (segment (start 139.7 93.98) (end 147.32 93.98) (width 0.25) (layer B.Cu) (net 5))
 (via (at 139.7 93.98) (size 0.6) (drill 0.4) (layers F.Cu B.Cu) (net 5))
 (segment (start 139.7 93.98) (end 139.7 86.36) (width 0.25) (layer F.Cu) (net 5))
 (segment (start 190.5 101.6) (end 190.5 104.14) (width 0.25) (layer B.Cu) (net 5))
 (segment (start 147.32 99.06) (end 147.32 104.14) (width 0.25) (layer B.Cu) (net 5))
 (segment (start 157.48 99.06) (end 147.32 99.06) (width 0.25) (layer B.Cu) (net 5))
 (via (at 157.48 99.06) (size 0.6) (drill 0.4) (layers F.Cu B.Cu) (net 5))
 (segment (start 157.48 104.14) (end 157.48 99.06) (width 0.25) (layer F.Cu) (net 5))
 (via (at 157.48 104.14) (size 0.6) (drill 0.4) (layers F.Cu B.Cu) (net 5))
 (segment (start 185.42 104.14) (end 157.48 104.14) (width 0.25) (layer B.Cu) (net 5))
 (via (at 185.42 104.14) (size 0.6) (drill 0.4) (layers F.Cu B.Cu) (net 5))
 (segment (start 190.5 104.14) (end 185.42 104.14) (width 0.25) (layer F.Cu) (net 5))
 (via (at 190.5 104.14) (size 0.6) (drill 0.4) (layers F.Cu B.Cu) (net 5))
 (segment (start 139.7 86.36) (end 144.78 86.36) (width 0.25) (layer B.Cu) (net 5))
 (segment (start 139.7 83.82) (end 139.7 86.36) (width 0.25) (layer B.Cu) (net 5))
 (segment (start 190.5 101.6) (end 190.5 96.52) (width 0.25) (layer B.Cu) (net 5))
 (segment (start 162.56 66.04) (end 162.56 73.66) (width 0.25) (layer B.Cu) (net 6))
 (segment (start 162.56 66.04) (end 172.72 66.04) (width 0.25) (layer B.Cu) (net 6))
 (segment (start 137.16 73.66) (end 162.56 73.66) (width 0.25) (layer B.Cu) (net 6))
 (segment (start 172.72 83.82) (end 172.72 88.9) (width 0.25) (layer B.Cu) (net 6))
 (via (at 187.96 88.9) (size 0.6) (drill 0.4) (layers F.Cu B.Cu) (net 6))
 (segment (start 175.26 88.9) (end 187.96 88.9) (width 0.25) (layer F.Cu) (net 6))
 (via (at 175.26 88.9) (size 0.6) (drill 0.4) (layers F.Cu B.Cu) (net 6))
 (segment (start 172.72 88.9) (end 175.26 88.9) (width 0.25) (layer B.Cu) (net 6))
 (segment (start 187.96 96.52) (end 187.96 88.9) (width 0.25) (layer B.Cu) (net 6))
 (segment (start 187.96 88.9) (end 187.96 86.36) (width 0.25) (layer B.Cu) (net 6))
 (segment (start 187.96 86.36) (end 187.96 81.28) (width 0.25) (layer B.Cu) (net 6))
 (segment (start 187.96 81.28) (end 200.66 81.28) (width 0.25) (layer B.Cu) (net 6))
 (segment (start 162.56 73.66) (end 162.56 83.82) (width 0.25) (layer B.Cu) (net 6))
 (segment (start 162.56 83.82) (end 172.72 83.82) (width 0.25) (layer B.Cu) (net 6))
 (segment (start 172.72 83.82) (end 175.26 83.82) (width 0.25) (layer B.Cu) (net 6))
 (segment (start 134.62 88.9) (end 134.62 73.66) (width 0.25) (layer B.Cu) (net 6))
 (segment (start 134.62 73.66) (end 137.16 73.66) (width 0.25) (layer B.Cu) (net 6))
 (segment (start 185.42 86.36) (end 187.96 86.36) (width 0.25) (layer B.Cu) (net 6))
 (segment (start 203.2 68.66) (end 203.2 66.04) (width 0.25) (layer B.Cu) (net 17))
 (segment (start 203.2 66.04) (end 182.88 66.04) (width 0.25) (layer B.Cu) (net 17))
 (segment (start 205.74 81.28) (end 205.74 68.58) (width 0.25) (layer B.Cu) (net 17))
 (segment (start 205.66 68.66) (end 203.2 68.66) (width 0.25) (layer B.Cu) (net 17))
 (segment (start 205.74 68.58) (end 205.66 68.66) (width 0.25) (layer B.Cu) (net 17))
 (via (at 182.88 66.04) (size 0.6) (drill 0.4) (layers F.Cu B.Cu) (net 17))
 (segment (start 170.18 96.52) (end 170.18 93.98) (width 0.25) (layer B.Cu) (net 12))
 (segment (start 170.18 81.28) (end 175.26 81.28) (width 0.25) (layer B.Cu) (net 12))
 (via (at 170.18 81.28) (size 0.6) (drill 0.4) (layers F.Cu B.Cu) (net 12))
 (segment (start 170.18 93.98) (end 170.18 81.28) (width 0.25) (layer F.Cu) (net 12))
 (via (at 170.18 93.98) (size 0.6) (drill 0.4) (layers F.Cu B.Cu) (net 12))
 (segment (start 170.18 99.06) (end 170.18 96.52) (width 0.25) (layer B.Cu) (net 12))
 (segment (start 175.26 66.04) (end 175.26 63.5) (width 0.25) (layer B.Cu) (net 16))
 (segment (start 172.72 63.5) (end 175.26 63.5) (width 0.25) (layer B.Cu) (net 16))
 (segment (start 195.58 53.34) (end 195.58 63.5) (width 0.25) (layer B.Cu) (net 19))
 (segment (start 195.58 78.74) (end 182.88 78.74) (width 0.25) (layer B.Cu) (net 19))
 (via (at 195.58 78.74) (size 0.6) (drill 0.4) (layers F.Cu B.Cu) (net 19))
 (segment (start 195.58 63.5) (end 195.58 78.74) (width 0.25) (layer F.Cu) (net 19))
 (via (at 195.58 63.5) (size 0.6) (drill 0.4) (layers F.Cu B.Cu) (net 19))
 (segment (start 185.42 53.34) (end 185.42 63.5) (width 0.25) (layer B.Cu) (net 3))
 (segment (start 185.42 71.12) (end 182.88 71.12) (width 0.25) (layer B.Cu) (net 3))
 (via (at 185.42 71.12) (size 0.6) (drill 0.4) (layers F.Cu B.Cu) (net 3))
 (segment (start 185.42 63.5) (end 185.42 71.12) (width 0.25) (layer F.Cu) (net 3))
 (via (at 185.42 63.5) (size 0.6) (drill 0.4) (layers F.Cu B.Cu) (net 3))
 (segment (start 175.26 53.34) (end 177.8 53.34) (width 0.25) (layer B.Cu) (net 4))
 (segment (start 177.8 71.12) (end 175.26 71.12) (width 0.25) (layer B.Cu) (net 4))
 (segment (start 177.8 53.34) (end 177.8 71.12) (width 0.25) (layer B.Cu) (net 4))
 (segment (start 165.1 53.34) (end 165.1 60.96) (width 0.25) (layer B.Cu) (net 1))
 (segment (start 165.1 78.74) (end 175.26 78.74) (width 0.25) (layer B.Cu) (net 1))
 (via (at 165.1 78.74) (size 0.6) (drill 0.4) (layers F.Cu B.Cu) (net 1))
 (segment (start 165.1 60.96) (end 165.1 78.74) (width 0.25) (layer F.Cu) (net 1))
 (via (at 165.1 60.96) (size 0.6) (drill 0.4) (layers F.Cu B.Cu) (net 1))
 (segment (start 137.16 83.82) (end 137.16 81.28) (width 0.25) (layer B.Cu) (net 18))
 (segment (start 134.62 93.98) (end 137.16 93.98) (width 0.25) (layer B.Cu) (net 18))
 (segment (start 137.16 86.36) (end 137.16 83.82) (width 0.25) (layer B.Cu) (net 18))
 (via (at 137.16 86.36) (size 0.6) (drill 0.4) (layers F.Cu B.Cu) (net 18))
 (segment (start 137.16 93.98) (end 137.16 86.36) (width 0.25) (layer F.Cu) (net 18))
 (via (at 137.16 93.98) (size 0.6) (drill 0.4) (layers F.Cu B.Cu) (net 18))
 (segment (start 142.24 83.82) (end 142.24 78.74) (width 0.25) (layer B.Cu) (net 14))
 (segment (start 142.24 78.74) (end 144.78 78.74) (width 0.25) (layer B.Cu) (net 14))
 (segment (start 165.1 96.52) (end 165.1 88.9) (width 0.25) (layer B.Cu) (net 14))
 (segment (start 147.32 78.74) (end 144.78 78.74) (width 0.25) (layer B.Cu) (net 14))
 (segment (start 147.32 88.9) (end 147.32 78.74) (width 0.25) (layer B.Cu) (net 14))
 (segment (start 165.1 88.9) (end 147.32 88.9) (width 0.25) (layer B.Cu) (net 14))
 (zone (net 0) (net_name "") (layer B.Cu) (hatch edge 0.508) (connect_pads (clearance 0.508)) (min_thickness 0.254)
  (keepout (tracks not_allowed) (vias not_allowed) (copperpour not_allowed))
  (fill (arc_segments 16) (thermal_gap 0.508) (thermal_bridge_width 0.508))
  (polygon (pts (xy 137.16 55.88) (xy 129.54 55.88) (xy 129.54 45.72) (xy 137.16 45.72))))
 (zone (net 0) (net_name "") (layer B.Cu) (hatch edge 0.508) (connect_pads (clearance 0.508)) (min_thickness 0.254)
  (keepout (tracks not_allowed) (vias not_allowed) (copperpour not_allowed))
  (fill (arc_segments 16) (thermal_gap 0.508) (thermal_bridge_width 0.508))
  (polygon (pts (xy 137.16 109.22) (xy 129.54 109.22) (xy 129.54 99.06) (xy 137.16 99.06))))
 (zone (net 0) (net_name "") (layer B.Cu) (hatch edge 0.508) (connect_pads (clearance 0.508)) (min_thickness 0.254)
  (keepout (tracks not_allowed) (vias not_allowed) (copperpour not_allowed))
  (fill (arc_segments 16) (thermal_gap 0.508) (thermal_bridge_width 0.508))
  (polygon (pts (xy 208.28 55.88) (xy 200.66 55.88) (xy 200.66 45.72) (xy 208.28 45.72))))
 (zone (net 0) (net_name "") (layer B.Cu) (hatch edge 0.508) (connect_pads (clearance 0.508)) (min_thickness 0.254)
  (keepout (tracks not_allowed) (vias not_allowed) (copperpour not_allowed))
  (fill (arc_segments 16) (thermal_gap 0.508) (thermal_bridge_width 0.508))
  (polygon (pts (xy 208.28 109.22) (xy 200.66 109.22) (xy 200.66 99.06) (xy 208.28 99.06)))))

